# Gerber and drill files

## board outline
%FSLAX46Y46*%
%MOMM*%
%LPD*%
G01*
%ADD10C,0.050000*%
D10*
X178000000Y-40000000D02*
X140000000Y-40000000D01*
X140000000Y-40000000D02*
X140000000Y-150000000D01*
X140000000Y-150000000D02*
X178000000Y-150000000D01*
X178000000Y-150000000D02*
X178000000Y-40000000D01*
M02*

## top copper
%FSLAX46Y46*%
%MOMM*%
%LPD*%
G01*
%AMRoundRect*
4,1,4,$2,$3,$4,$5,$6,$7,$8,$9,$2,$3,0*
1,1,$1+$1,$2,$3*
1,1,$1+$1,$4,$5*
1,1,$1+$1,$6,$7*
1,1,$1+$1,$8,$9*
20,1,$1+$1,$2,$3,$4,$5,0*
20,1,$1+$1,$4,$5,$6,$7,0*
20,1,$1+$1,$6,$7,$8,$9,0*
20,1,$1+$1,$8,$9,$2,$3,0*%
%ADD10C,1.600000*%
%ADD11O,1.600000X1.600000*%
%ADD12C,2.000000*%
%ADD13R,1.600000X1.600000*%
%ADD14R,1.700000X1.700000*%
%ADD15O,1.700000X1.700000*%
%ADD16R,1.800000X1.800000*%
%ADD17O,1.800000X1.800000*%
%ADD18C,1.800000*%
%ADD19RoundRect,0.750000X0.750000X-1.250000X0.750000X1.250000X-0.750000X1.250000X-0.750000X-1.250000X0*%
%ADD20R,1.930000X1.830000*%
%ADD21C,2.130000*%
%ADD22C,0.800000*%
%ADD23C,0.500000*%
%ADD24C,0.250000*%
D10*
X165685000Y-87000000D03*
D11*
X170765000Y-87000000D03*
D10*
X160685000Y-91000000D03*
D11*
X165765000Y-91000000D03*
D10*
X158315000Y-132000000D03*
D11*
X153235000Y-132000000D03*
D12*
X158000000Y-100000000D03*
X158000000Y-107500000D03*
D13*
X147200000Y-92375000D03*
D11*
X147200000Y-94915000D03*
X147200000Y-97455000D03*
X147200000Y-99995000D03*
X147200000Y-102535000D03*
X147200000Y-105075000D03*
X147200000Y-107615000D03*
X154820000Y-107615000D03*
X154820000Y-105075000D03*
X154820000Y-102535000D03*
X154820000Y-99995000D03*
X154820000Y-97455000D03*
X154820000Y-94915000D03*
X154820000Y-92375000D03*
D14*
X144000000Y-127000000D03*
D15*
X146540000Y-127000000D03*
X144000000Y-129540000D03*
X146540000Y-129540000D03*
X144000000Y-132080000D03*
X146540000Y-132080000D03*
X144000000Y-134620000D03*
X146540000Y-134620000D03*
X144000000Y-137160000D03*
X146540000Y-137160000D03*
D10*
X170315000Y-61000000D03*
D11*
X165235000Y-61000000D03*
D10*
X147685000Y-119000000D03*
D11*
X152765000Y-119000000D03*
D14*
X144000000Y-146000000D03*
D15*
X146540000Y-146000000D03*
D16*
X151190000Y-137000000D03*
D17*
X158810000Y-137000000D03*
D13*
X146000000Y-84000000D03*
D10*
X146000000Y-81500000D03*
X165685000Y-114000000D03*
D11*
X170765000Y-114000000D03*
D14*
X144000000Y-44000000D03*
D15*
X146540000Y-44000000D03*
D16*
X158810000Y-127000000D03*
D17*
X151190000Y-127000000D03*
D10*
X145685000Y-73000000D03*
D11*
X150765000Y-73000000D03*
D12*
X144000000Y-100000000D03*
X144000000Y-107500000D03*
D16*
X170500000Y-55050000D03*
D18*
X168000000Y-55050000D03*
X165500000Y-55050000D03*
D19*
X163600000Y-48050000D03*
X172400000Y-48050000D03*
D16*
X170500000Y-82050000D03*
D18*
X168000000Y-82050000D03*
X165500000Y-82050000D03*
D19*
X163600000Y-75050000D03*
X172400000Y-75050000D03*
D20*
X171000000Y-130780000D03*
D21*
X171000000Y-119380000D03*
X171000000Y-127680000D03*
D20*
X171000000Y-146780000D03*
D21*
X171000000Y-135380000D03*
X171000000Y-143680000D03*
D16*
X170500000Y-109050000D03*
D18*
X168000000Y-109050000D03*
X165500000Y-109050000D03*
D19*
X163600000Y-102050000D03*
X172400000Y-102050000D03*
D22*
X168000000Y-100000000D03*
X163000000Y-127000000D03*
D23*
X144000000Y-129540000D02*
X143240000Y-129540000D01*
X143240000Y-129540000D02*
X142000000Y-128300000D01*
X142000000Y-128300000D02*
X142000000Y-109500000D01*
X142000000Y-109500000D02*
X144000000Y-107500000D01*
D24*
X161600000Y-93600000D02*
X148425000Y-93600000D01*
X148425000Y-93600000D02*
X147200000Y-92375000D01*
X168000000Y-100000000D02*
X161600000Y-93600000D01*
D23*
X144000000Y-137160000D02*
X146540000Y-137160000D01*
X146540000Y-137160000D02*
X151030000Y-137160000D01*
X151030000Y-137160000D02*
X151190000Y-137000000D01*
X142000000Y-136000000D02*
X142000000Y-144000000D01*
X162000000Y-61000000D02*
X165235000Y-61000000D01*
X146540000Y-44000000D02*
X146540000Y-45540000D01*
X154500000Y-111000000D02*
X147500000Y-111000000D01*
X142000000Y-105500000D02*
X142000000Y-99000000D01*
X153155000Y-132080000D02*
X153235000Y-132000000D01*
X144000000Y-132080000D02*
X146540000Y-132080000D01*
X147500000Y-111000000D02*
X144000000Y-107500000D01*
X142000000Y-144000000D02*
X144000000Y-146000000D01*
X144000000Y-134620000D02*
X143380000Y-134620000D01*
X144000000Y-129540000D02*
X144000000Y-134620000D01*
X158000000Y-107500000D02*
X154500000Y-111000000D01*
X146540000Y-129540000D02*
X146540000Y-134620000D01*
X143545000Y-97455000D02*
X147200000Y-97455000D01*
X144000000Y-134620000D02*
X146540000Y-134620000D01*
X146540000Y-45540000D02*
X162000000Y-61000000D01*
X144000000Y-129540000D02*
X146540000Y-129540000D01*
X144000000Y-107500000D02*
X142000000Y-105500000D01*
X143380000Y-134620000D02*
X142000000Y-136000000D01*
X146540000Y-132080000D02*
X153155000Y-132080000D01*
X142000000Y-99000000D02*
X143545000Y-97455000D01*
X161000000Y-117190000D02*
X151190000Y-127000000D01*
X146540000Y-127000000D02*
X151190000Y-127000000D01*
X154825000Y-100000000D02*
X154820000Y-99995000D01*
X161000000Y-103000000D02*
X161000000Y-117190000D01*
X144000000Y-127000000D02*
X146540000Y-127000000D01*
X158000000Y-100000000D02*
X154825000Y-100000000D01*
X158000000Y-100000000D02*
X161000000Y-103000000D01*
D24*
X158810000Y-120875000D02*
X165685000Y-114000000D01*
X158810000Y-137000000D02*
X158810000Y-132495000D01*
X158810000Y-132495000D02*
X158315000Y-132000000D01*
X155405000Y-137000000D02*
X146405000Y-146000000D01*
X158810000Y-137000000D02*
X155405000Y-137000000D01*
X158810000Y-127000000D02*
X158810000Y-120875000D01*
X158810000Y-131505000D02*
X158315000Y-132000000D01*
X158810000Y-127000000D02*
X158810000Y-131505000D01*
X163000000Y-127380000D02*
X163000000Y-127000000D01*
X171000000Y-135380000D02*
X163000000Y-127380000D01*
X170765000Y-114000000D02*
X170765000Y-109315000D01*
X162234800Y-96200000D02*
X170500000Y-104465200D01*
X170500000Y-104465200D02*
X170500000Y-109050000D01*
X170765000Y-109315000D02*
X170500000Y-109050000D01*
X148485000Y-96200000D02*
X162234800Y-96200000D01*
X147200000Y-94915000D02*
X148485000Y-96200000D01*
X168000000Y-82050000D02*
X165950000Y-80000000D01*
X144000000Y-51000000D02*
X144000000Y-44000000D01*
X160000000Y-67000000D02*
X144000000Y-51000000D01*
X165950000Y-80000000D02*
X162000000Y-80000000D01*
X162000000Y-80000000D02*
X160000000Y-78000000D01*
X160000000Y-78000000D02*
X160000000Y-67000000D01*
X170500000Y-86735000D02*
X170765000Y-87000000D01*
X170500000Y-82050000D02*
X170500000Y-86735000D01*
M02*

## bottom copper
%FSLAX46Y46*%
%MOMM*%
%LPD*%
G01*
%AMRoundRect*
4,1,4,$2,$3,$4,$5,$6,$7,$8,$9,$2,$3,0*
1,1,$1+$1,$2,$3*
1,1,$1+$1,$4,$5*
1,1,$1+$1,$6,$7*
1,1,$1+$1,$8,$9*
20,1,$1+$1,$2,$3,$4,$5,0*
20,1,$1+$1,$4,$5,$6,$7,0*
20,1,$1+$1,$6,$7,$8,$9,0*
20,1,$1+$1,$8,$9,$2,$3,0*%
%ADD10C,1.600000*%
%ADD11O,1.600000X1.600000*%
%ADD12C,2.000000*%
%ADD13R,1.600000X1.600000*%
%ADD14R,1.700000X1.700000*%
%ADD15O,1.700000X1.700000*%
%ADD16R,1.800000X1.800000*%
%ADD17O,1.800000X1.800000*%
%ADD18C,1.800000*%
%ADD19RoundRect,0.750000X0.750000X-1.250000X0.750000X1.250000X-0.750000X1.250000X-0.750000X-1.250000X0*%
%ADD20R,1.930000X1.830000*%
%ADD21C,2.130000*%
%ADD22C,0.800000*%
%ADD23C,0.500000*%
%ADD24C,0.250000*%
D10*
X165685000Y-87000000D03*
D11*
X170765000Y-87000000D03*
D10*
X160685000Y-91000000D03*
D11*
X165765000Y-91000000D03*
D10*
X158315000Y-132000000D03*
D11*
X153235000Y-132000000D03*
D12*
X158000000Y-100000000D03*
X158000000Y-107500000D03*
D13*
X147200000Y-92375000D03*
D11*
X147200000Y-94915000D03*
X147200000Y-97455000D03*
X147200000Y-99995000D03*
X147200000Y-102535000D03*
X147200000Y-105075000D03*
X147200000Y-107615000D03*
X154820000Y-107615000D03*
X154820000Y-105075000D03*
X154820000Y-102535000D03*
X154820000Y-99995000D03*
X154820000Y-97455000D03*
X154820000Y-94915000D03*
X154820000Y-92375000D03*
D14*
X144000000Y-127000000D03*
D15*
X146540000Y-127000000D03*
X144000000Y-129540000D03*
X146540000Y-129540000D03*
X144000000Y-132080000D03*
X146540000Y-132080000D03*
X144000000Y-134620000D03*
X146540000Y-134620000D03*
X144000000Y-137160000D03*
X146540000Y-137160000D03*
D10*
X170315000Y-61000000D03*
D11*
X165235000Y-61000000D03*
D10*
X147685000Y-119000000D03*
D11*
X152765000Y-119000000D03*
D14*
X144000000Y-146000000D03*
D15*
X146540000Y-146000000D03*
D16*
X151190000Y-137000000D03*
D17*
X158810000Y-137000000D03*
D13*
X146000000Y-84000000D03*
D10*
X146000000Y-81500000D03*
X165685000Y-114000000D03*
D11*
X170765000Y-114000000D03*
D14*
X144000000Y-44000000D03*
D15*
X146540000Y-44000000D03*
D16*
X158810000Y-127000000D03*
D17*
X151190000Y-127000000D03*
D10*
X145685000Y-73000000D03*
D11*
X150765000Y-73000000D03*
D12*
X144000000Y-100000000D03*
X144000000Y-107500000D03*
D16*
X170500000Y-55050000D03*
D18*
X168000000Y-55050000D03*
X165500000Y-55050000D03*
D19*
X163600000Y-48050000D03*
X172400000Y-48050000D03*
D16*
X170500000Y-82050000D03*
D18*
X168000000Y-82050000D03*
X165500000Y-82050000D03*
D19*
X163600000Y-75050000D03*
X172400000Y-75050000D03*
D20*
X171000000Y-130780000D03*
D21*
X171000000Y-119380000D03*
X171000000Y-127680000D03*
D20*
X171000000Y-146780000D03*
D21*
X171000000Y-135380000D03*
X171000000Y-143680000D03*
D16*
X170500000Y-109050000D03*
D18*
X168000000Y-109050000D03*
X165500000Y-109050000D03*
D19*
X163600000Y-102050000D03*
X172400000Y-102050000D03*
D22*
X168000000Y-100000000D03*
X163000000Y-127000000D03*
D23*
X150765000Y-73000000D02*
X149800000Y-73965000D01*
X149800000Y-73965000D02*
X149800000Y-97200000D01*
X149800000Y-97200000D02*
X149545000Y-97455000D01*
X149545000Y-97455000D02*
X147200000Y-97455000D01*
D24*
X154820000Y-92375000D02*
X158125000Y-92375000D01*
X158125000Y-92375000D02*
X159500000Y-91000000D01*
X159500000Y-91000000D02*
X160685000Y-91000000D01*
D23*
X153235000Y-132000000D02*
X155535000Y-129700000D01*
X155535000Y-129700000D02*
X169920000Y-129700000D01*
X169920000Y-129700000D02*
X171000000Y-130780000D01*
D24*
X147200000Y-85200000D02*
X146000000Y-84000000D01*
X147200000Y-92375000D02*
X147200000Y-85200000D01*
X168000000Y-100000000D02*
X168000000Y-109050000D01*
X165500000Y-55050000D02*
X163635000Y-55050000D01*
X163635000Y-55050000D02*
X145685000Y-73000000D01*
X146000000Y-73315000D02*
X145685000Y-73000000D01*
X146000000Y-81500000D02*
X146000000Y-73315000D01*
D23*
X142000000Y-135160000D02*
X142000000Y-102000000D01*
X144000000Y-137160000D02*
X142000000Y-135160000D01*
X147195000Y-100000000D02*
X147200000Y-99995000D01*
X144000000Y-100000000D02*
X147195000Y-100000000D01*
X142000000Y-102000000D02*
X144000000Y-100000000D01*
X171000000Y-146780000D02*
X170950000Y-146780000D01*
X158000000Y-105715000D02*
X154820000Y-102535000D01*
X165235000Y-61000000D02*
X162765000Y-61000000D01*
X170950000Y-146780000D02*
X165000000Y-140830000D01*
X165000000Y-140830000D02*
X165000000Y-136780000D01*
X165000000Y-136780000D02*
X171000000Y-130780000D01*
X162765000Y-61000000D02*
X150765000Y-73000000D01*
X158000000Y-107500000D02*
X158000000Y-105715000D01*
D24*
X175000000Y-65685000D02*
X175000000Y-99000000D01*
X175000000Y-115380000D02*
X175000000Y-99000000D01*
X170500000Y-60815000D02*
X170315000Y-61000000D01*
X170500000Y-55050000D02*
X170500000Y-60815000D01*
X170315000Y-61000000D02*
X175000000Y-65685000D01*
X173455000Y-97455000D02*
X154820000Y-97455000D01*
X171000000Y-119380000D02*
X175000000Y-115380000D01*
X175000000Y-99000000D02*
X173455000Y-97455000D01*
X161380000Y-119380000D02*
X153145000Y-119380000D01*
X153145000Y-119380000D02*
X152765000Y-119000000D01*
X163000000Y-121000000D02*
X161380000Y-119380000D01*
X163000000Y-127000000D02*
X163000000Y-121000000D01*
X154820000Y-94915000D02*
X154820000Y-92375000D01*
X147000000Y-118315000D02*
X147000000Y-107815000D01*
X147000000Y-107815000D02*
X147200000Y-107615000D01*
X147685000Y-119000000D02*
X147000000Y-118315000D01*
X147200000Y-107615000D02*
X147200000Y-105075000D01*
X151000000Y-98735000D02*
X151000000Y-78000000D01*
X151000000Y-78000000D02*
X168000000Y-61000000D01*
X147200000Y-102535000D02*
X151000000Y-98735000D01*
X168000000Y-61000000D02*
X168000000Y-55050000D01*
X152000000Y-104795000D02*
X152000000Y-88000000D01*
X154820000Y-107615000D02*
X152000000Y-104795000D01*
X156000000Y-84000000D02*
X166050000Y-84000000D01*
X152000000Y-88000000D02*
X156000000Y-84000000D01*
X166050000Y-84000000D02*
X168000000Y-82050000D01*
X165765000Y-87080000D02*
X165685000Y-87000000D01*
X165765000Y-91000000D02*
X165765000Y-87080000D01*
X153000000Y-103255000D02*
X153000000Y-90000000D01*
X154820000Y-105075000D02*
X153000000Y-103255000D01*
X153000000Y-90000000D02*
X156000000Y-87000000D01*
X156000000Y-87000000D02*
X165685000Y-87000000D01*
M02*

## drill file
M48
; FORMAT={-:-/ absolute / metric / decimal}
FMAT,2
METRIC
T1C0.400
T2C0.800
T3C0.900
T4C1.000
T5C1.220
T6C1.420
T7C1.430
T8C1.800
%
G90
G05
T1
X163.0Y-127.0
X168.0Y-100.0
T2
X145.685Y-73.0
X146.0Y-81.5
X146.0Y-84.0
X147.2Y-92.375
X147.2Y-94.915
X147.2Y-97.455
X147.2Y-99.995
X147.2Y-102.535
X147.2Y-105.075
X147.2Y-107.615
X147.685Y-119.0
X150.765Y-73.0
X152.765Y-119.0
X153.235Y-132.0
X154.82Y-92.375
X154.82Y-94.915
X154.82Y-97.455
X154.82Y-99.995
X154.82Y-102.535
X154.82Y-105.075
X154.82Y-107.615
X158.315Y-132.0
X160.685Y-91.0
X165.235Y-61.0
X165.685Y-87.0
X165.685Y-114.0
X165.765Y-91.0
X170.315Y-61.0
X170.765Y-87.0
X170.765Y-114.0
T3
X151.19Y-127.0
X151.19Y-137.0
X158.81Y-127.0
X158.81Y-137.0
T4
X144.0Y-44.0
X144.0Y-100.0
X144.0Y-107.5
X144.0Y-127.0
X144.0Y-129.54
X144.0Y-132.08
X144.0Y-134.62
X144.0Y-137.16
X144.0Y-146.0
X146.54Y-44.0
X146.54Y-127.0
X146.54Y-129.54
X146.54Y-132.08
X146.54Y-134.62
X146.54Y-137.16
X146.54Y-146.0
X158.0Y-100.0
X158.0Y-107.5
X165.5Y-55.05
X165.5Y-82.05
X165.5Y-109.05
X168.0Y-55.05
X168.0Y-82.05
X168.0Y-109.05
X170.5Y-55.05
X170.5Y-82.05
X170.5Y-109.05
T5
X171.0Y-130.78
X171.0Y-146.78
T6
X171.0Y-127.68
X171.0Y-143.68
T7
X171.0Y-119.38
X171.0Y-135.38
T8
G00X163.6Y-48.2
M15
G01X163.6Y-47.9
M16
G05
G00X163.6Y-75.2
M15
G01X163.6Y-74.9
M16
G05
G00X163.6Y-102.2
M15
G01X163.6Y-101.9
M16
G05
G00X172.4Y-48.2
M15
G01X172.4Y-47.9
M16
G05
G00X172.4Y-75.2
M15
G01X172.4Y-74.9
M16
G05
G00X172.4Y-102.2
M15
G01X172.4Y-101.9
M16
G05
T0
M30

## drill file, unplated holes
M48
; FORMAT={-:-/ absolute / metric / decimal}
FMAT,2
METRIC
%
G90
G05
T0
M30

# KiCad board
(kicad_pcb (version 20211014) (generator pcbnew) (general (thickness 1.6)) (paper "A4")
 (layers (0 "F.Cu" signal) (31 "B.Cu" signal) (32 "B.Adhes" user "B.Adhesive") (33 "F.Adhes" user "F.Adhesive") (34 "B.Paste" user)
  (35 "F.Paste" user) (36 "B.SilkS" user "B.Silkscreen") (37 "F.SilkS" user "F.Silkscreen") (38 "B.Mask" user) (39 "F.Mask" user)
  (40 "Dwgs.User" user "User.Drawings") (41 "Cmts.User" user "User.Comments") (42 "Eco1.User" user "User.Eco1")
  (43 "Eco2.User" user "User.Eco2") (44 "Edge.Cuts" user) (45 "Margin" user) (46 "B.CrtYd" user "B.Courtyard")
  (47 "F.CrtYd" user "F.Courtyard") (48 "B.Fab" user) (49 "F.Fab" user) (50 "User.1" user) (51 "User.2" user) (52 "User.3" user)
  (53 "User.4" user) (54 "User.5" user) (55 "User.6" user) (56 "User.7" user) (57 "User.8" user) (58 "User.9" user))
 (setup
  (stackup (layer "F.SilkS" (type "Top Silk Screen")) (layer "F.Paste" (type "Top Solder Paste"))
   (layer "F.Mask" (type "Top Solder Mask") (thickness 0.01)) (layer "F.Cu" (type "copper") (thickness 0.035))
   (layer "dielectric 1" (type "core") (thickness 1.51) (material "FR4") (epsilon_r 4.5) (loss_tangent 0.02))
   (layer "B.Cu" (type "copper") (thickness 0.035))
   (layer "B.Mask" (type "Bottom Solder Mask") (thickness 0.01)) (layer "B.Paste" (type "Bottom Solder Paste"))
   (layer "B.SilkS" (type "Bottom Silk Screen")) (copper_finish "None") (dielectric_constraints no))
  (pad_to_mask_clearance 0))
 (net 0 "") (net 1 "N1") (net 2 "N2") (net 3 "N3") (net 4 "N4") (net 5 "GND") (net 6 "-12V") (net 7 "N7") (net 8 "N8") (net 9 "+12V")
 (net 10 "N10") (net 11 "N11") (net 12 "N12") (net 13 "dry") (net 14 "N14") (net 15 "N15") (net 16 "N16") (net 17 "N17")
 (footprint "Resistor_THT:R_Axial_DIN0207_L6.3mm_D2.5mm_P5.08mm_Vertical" (layer "F.Cu") (at 165.685 87)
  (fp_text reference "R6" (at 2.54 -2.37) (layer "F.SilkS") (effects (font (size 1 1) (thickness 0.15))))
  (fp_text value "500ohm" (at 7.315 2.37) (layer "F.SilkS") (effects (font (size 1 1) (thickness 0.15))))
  (pad "1" thru_hole circle (at 0 0) (size 1.6 1.6) (drill 0.8) (layers *.Cu *.Mask) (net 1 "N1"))
  (pad "2" thru_hole oval (at 5.08 0) (size 1.6 1.6) (drill 0.8) (layers *.Cu *.Mask) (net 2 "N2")))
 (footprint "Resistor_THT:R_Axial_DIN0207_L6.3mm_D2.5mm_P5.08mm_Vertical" (layer "F.Cu") (at 160.685 91)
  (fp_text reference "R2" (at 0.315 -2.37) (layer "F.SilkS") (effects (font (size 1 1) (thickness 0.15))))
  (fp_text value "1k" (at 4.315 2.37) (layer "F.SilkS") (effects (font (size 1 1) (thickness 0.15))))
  (pad "1" thru_hole circle (at 0 0) (size 1.6 1.6) (drill 0.8) (layers *.Cu *.Mask) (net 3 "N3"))
  (pad "2" thru_hole oval (at 5.08 0) (size 1.6 1.6) (drill 0.8) (layers *.Cu *.Mask) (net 1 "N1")))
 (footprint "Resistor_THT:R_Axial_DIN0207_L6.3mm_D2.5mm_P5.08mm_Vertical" (layer "F.Cu") (at 158.315 132 180)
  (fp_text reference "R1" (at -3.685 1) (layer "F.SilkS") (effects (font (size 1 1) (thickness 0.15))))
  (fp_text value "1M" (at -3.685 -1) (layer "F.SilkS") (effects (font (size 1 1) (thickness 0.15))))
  (pad "1" thru_hole circle (at 0 0 180) (size 1.6 1.6) (drill 0.8) (layers *.Cu *.Mask) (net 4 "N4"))
  (pad "2" thru_hole oval (at 5.08 0 180) (size 1.6 1.6) (drill 0.8) (layers *.Cu *.Mask) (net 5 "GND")))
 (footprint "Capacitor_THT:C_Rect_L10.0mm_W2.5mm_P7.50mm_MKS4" (layer "F.Cu") (at 158 100 -90)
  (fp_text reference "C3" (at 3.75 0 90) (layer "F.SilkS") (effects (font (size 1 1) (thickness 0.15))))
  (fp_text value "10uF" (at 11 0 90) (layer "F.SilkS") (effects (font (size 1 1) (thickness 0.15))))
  (pad "1" thru_hole circle (at 0 0 270) (size 2 2) (drill 1) (layers *.Cu *.Mask) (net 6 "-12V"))
  (pad "2" thru_hole circle (at 7.5 0 270) (size 2 2) (drill 1) (layers *.Cu *.Mask) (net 5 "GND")))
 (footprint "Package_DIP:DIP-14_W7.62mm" (layer "F.Cu") (at 147.2 92.375)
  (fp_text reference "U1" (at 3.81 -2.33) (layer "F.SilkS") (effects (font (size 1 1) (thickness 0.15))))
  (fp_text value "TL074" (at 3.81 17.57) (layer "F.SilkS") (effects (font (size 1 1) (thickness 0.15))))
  (pad "1" thru_hole rect (at 0 0) (size 1.6 1.6) (drill 0.8) (layers *.Cu *.Mask) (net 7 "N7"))
  (pad "2" thru_hole oval (at 0 2.54) (size 1.6 1.6) (drill 0.8) (layers *.Cu *.Mask) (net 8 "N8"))
  (pad "3" thru_hole oval (at 0 5.08) (size 1.6 1.6) (drill 0.8) (layers *.Cu *.Mask) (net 5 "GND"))
  (pad "4" thru_hole oval (at 0 7.62) (size 1.6 1.6) (drill 0.8) (layers *.Cu *.Mask) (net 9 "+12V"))
  (pad "5" thru_hole oval (at 0 10.16) (size 1.6 1.6) (drill 0.8) (layers *.Cu *.Mask) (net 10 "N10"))
  (pad "6" thru_hole oval (at 0 12.7) (size 1.6 1.6) (drill 0.8) (layers *.Cu *.Mask) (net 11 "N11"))
  (pad "7" thru_hole oval (at 0 15.24) (size 1.6 1.6) (drill 0.8) (layers *.Cu *.Mask) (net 11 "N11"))
  (pad "8" thru_hole oval (at 7.62 15.24) (size 1.6 1.6) (drill 0.8) (layers *.Cu *.Mask) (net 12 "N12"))
  (pad "9" thru_hole oval (at 7.62 12.7) (size 1.6 1.6) (drill 0.8) (layers *.Cu *.Mask) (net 1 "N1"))
  (pad "10" thru_hole oval (at 7.62 10.16) (size 1.6 1.6) (drill 0.8) (layers *.Cu *.Mask) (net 5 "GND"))
  (pad "11" thru_hole oval (at 7.62 7.62) (size 1.6 1.6) (drill 0.8) (layers *.Cu *.Mask) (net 6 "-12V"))
  (pad "12" thru_hole oval (at 7.62 5.08) (size 1.6 1.6) (drill 0.8) (layers *.Cu *.Mask) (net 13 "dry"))
  (pad "13" thru_hole oval (at 7.62 2.54) (size 1.6 1.6) (drill 0.8) (layers *.Cu *.Mask) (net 3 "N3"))
  (pad "14" thru_hole oval (at 7.62 0) (size 1.6 1.6) (drill 0.8) (layers *.Cu *.Mask) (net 3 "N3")))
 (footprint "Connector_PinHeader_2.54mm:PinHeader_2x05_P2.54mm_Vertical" (layer "F.Cu") (at 144 127)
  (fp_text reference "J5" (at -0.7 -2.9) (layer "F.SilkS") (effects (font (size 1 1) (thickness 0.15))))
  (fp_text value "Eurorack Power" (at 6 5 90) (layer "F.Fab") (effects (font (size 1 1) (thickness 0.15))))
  (pad "1" thru_hole rect (at 0 0) (size 1.7 1.7) (drill 1) (layers *.Cu *.Mask) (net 6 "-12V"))
  (pad "2" thru_hole oval (at 2.54 0) (size 1.7 1.7) (drill 1) (layers *.Cu *.Mask) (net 6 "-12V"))
  (pad "3" thru_hole oval (at 0 2.54) (size 1.7 1.7) (drill 1) (layers *.Cu *.Mask) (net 5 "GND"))
  (pad "4" thru_hole oval (at 2.54 2.54) (size 1.7 1.7) (drill 1) (layers *.Cu *.Mask) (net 5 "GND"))
  (pad "5" thru_hole oval (at 0 5.08) (size 1.7 1.7) (drill 1) (layers *.Cu *.Mask) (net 5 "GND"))
  (pad "6" thru_hole oval (at 2.54 5.08) (size 1.7 1.7) (drill 1) (layers *.Cu *.Mask) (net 5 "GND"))
  (pad "7" thru_hole oval (at 0 7.62) (size 1.7 1.7) (drill 1) (layers *.Cu *.Mask) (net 5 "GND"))
  (pad "8" thru_hole oval (at 2.54 7.62) (size 1.7 1.7) (drill 1) (layers *.Cu *.Mask) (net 5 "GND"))
  (pad "9" thru_hole oval (at 0 10.16) (size 1.7 1.7) (drill 1) (layers *.Cu *.Mask) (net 9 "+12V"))
  (pad "10" thru_hole oval (at 2.54 10.16) (size 1.7 1.7) (drill 1) (layers *.Cu *.Mask) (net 9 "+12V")))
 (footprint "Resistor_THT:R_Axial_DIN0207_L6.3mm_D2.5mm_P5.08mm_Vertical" (layer "F.Cu") (at 170.315 61 180)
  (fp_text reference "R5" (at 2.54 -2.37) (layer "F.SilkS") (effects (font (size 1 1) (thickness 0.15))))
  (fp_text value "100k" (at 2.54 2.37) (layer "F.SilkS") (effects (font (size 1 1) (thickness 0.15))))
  (pad "1" thru_hole circle (at 0 0 180) (size 1.6 1.6) (drill 0.8) (layers *.Cu *.Mask) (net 13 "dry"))
  (pad "2" thru_hole oval (at 5.08 0 180) (size 1.6 1.6) (drill 0.8) (layers *.Cu *.Mask) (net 5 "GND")))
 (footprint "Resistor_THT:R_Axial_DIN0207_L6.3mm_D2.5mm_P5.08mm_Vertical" (layer "F.Cu") (at 147.685 119)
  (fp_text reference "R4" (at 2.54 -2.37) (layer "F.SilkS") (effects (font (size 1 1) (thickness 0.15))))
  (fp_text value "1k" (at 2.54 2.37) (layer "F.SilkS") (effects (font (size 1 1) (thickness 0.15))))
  (pad "1" thru_hole circle (at 0 0) (size 1.6 1.6) (drill 0.8) (layers *.Cu *.Mask) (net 11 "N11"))
  (pad "2" thru_hole oval (at 5.08 0) (size 1.6 1.6) (drill 0.8) (layers *.Cu *.Mask) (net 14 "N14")))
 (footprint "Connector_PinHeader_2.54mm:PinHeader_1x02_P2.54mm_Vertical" (layer "F.Cu") (at 144 146 90)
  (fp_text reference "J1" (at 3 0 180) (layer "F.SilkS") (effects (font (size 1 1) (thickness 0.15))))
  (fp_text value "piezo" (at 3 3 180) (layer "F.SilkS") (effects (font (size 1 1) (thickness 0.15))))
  (pad "1" thru_hole rect (at 0 0 90) (size 1.7 1.7) (drill 1) (layers *.Cu *.Mask) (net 5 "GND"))
  (pad "2" thru_hole oval (at 0 2.54 90) (size 1.7 1.7) (drill 1) (layers *.Cu *.Mask) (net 4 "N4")))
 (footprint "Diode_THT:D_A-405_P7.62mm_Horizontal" (layer "F.Cu") (at 151.19 137)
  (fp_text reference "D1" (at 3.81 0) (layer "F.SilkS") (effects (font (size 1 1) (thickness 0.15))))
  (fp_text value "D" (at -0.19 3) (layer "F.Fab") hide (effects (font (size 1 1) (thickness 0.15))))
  (pad "1" thru_hole rect (at 0 0) (size 1.8 1.8) (drill 0.9) (layers *.Cu *.Mask) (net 9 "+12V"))
  (pad "2" thru_hole oval (at 7.62 0) (size 1.8 1.8) (drill 0.9) (layers *.Cu *.Mask) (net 4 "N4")))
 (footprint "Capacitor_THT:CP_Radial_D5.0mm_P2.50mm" (layer "F.Cu") (at 146 84 90)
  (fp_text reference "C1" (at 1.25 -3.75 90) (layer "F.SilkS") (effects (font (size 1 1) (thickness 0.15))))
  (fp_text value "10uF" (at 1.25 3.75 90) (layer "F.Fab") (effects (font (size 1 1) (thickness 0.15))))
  (pad "1" thru_hole rect (at 0 0 90) (size 1.6 1.6) (drill 0.8) (layers *.Cu *.Mask) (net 7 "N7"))
  (pad "2" thru_hole circle (at 2.5 0 90) (size 1.6 1.6) (drill 0.8) (layers *.Cu *.Mask) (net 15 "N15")))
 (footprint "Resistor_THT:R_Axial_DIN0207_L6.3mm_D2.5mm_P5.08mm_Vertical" (layer "F.Cu") (at 165.685 114)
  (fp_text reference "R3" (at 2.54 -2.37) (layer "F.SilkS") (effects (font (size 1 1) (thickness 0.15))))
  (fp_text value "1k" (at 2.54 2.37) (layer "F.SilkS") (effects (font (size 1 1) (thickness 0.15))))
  (pad "1" thru_hole circle (at 0 0) (size 1.6 1.6) (drill 0.8) (layers *.Cu *.Mask) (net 4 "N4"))
  (pad "2" thru_hole oval (at 5.08 0) (size 1.6 1.6) (drill 0.8) (layers *.Cu *.Mask) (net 8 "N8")))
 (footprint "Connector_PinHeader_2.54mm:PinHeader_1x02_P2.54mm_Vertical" (layer "F.Cu") (at 144 44 90)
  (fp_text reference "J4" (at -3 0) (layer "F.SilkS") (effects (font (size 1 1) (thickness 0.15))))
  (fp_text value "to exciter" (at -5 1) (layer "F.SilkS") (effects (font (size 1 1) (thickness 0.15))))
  (pad "1" thru_hole rect (at 0 0 90) (size 1.7 1.7) (drill 1) (layers *.Cu *.Mask) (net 12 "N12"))
  (pad "2" thru_hole oval (at 0 2.54 90) (size 1.7 1.7) (drill 1) (layers *.Cu *.Mask) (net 5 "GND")))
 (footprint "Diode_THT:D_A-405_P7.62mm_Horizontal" (layer "F.Cu") (at 158.81 127 180)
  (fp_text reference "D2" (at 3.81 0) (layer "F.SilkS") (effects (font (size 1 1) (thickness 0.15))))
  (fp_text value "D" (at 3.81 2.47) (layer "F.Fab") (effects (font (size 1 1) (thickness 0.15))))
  (pad "1" thru_hole rect (at 0 0 180) (size 1.8 1.8) (drill 0.9) (layers *.Cu *.Mask) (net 4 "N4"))
  (pad "2" thru_hole oval (at 7.62 0 180) (size 1.8 1.8) (drill 0.9) (layers *.Cu *.Mask) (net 6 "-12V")))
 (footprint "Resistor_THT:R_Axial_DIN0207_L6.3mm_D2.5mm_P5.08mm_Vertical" (layer "F.Cu") (at 145.685 73)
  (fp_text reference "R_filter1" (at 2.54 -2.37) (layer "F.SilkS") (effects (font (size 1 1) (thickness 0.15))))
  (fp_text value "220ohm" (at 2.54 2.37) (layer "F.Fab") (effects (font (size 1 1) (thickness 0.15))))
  (pad "1" thru_hole circle (at 0 0) (size 1.6 1.6) (drill 0.8) (layers *.Cu *.Mask) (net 15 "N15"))
  (pad "2" thru_hole oval (at 5.08 0) (size 1.6 1.6) (drill 0.8) (layers *.Cu *.Mask) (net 5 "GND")))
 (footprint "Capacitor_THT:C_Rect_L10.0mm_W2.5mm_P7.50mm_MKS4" (layer "F.Cu") (at 144 100 -90)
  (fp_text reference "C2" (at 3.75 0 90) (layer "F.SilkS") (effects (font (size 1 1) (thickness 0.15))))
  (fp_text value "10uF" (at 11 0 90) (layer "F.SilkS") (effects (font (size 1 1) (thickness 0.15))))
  (pad "1" thru_hole circle (at 0 0 270) (size 2 2) (drill 1) (layers *.Cu *.Mask) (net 9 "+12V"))
  (pad "2" thru_hole circle (at 7.5 0 270) (size 2 2) (drill 1) (layers *.Cu *.Mask) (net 5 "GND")))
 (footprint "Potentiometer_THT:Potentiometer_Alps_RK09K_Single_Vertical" (layer "B.Cu") (at 170.5 55.05 90)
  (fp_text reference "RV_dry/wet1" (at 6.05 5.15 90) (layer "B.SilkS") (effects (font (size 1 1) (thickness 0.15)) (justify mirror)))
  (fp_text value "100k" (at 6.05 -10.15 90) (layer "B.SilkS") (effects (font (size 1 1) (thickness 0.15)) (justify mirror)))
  (pad "1" thru_hole rect (at 0 0 90) (size 1.8 1.8) (drill 1) (layers *.Cu *.Mask) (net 13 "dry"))
  (pad "2" thru_hole circle (at 0 -2.5 90) (size 1.8 1.8) (drill 1) (layers *.Cu *.Mask) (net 10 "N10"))
  (pad "3" thru_hole circle (at 0 -5 90) (size 1.8 1.8) (drill 1) (layers *.Cu *.Mask) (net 15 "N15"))
  (pad "MP" thru_hole roundrect (at 7 -6.9 90) (size 4 3) (drill oval 2.1 1.8) (layers *.Cu *.Mask) (roundrect_rratio 0.25))
  (pad "MP" thru_hole roundrect (at 7 1.9 90) (size 4 3) (drill oval 2.1 1.8) (layers *.Cu *.Mask) (roundrect_rratio 0.25)))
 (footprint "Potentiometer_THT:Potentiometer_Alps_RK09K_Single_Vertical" (layer "B.Cu") (at 170.5 82.05 90)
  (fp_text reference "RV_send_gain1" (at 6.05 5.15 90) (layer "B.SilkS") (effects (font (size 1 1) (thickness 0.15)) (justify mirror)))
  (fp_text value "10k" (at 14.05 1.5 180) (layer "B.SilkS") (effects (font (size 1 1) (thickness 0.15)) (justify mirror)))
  (pad "1" thru_hole rect (at 0 0 90) (size 1.8 1.8) (drill 1) (layers *.Cu *.Mask) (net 2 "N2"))
  (pad "2" thru_hole circle (at 0 -2.5 90) (size 1.8 1.8) (drill 1) (layers *.Cu *.Mask) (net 12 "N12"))
  (pad "3" thru_hole circle (at 0 -5 90) (size 1.8 1.8) (drill 1) (layers *.Cu *.Mask))
  (pad "MP" thru_hole roundrect (at 7 -6.9 90) (size 4 3) (drill oval 2.1 1.8) (layers *.Cu *.Mask) (roundrect_rratio 0.25))
  (pad "MP" thru_hole roundrect (at 7 1.9 90) (size 4 3) (drill oval 2.1 1.8) (layers *.Cu *.Mask) (roundrect_rratio 0.25)))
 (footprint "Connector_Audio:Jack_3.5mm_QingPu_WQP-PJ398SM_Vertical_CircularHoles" (layer "B.Cu") (at 171 130.78)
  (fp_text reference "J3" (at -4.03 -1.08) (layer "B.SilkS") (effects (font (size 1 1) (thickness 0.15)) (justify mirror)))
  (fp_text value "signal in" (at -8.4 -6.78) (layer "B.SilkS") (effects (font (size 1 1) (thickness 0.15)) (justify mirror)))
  (pad "S" thru_hole rect (at 0 0 180) (size 1.93 1.83) (drill 1.22) (layers *.Cu *.Mask) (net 5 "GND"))
  (pad "T" thru_hole circle (at 0 -11.4 180) (size 2.13 2.13) (drill 1.43) (layers *.Cu *.Mask) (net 13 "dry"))
  (pad "TN" thru_hole circle (at 0 -3.1 180) (size 2.13 2.13) (drill 1.42) (layers *.Cu *.Mask) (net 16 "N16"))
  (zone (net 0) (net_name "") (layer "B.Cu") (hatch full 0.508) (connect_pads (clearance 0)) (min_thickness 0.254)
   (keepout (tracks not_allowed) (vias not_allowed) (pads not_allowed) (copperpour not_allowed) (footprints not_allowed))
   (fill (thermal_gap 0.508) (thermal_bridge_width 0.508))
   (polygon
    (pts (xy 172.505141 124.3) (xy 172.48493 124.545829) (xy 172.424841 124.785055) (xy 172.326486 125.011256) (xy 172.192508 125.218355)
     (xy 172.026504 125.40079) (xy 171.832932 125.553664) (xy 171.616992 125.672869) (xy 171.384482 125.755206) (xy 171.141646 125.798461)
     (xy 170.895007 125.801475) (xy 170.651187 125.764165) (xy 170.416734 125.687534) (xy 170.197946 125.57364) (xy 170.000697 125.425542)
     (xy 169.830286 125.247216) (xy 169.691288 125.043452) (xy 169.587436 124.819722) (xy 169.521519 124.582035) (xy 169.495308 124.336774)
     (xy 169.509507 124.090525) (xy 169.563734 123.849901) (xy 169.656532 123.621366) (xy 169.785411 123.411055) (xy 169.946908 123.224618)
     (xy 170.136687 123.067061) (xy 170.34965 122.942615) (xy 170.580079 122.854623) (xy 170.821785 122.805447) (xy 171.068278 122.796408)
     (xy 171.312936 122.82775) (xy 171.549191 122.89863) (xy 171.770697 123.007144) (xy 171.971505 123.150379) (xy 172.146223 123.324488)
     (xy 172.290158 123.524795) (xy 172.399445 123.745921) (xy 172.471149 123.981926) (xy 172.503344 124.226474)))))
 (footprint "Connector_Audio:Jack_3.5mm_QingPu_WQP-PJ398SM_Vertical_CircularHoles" (layer "B.Cu") (at 171 146.78)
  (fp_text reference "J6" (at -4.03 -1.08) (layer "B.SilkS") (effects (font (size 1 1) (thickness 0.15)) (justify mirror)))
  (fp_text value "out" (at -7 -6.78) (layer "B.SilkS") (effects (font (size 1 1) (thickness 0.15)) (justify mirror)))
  (pad "S" thru_hole rect (at 0 0 180) (size 1.93 1.83) (drill 1.22) (layers *.Cu *.Mask) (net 5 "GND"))
  (pad "T" thru_hole circle (at 0 -11.4 180) (size 2.13 2.13) (drill 1.43) (layers *.Cu *.Mask) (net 14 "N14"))
  (pad "TN" thru_hole circle (at 0 -3.1 180) (size 2.13 2.13) (drill 1.42) (layers *.Cu *.Mask) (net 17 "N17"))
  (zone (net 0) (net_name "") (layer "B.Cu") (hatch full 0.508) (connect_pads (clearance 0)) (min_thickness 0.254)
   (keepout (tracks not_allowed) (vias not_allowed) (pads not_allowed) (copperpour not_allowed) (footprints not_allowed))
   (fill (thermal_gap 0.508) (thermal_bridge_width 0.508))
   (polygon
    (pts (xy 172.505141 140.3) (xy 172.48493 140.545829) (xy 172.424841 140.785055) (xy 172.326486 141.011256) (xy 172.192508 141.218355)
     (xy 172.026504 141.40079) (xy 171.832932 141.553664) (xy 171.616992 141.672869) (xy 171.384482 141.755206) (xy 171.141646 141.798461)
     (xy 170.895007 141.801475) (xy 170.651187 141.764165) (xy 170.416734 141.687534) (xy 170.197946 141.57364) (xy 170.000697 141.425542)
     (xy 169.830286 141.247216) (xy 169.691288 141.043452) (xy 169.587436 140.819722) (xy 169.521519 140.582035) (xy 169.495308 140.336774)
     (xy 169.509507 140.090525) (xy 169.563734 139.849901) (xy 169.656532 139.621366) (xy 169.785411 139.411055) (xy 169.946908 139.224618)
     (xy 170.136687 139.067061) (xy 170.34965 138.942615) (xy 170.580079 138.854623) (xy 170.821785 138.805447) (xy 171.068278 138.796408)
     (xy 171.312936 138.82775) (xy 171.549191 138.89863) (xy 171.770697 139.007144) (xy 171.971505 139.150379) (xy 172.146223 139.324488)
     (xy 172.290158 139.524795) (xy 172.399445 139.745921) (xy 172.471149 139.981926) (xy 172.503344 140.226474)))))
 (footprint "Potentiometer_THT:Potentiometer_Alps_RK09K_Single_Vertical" (layer "B.Cu") (at 170.5 109.05 90)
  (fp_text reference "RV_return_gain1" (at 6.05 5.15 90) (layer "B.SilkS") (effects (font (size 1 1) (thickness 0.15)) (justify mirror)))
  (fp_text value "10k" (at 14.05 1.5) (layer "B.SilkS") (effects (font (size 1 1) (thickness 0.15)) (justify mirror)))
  (pad "1" thru_hole rect (at 0 0 90) (size 1.8 1.8) (drill 1) (layers *.Cu *.Mask) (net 8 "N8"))
  (pad "2" thru_hole circle (at 0 -2.5 90) (size 1.8 1.8) (drill 1) (layers *.Cu *.Mask) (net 7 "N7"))
  (pad "3" thru_hole circle (at 0 -5 90) (size 1.8 1.8) (drill 1) (layers *.Cu *.Mask))
  (pad "MP" thru_hole roundrect (at 7 -6.9 90) (size 4 3) (drill oval 2.1 1.8) (layers *.Cu *.Mask) (roundrect_rratio 0.25))
  (pad "MP" thru_hole roundrect (at 7 1.9 90) (size 4 3) (drill oval 2.1 1.8) (layers *.Cu *.Mask) (roundrect_rratio 0.25)))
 (gr_rect (start 178 40) (end 140 150) (layer "Edge.Cuts") (width 0.05) (fill none))
 (segment (start 161.6 93.6) (end 148.425 93.6) (width 0.25) (layer "F.Cu") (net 7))
 (segment (start 148.425 93.6) (end 147.2 92.375) (width 0.25) (layer "F.Cu") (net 7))
 (segment (start 168 100) (end 161.6 93.6) (width 0.25) (layer "F.Cu") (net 7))
 (via (at 168 100) (size 0.8) (drill 0.4) (layers "F.Cu" "B.Cu") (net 7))
 (segment (start 147.2 85.2) (end 146 84) (width 0.25) (layer "B.Cu") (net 7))
 (segment (start 147.2 92.375) (end 147.2 85.2) (width 0.25) (layer "B.Cu") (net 7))
 (segment (start 168 100) (end 168 109.05) (width 0.25) (layer "B.Cu") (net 7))
 (segment (start 165.5 55.05) (end 163.635 55.05) (width 0.25) (layer "B.Cu") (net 15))
 (segment (start 163.635 55.05) (end 145.685 73) (width 0.25) (layer "B.Cu") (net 15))
 (segment (start 146 73.315) (end 145.685 73) (width 0.25) (layer "B.Cu") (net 15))
 (segment (start 146 81.5) (end 146 73.315) (width 0.25) (layer "B.Cu") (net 15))
 (segment (start 144 137.16) (end 146.54 137.16) (width 0.5) (layer "F.Cu") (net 9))
 (segment (start 146.54 137.16) (end 151.03 137.16) (width 0.5) (layer "F.Cu") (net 9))
 (segment (start 151.03 137.16) (end 151.19 137) (width 0.5) (layer "F.Cu") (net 9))
 (segment (start 142 135.16) (end 142 102) (width 0.5) (layer "B.Cu") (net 9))
 (segment (start 144 137.16) (end 142 135.16) (width 0.5) (layer "B.Cu") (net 9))
 (segment (start 147.195 100) (end 147.2 99.995) (width 0.5) (layer "B.Cu") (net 9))
 (segment (start 144 100) (end 147.195 100) (width 0.5) (layer "B.Cu") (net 9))
 (segment (start 142 102) (end 144 100) (width 0.5) (layer "B.Cu") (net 9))
 (segment (start 142 109.5) (end 144 107.5) (width 0.5) (layer "F.Cu") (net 5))
 (segment (start 142 136) (end 142 144) (width 0.5) (layer "F.Cu") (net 5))
 (segment (start 162 61) (end 165.235 61) (width 0.5) (layer "F.Cu") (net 5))
 (segment (start 146.54 44) (end 146.54 45.54) (width 0.5) (layer "F.Cu") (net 5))
 (segment (start 154.5 111) (end 147.5 111) (width 0.5) (layer "F.Cu") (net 5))
 (segment (start 142 105.5) (end 142 99) (width 0.5) (layer "F.Cu") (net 5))
 (segment (start 153.155 132.08) (end 153.235 132) (width 0.5) (layer "F.Cu") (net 5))
 (segment (start 144 132.08) (end 146.54 132.08) (width 0.5) (layer "F.Cu") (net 5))
 (segment (start 147.5 111) (end 144 107.5) (width 0.5) (layer "F.Cu") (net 5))
 (segment (start 142 144) (end 144 146) (width 0.5) (layer "F.Cu") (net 5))
 (segment (start 144 134.62) (end 143.38 134.62) (width 0.5) (layer "F.Cu") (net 5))
 (segment (start 144 129.54) (end 144 134.62) (width 0.5) (layer "F.Cu") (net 5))
 (segment (start 158 107.5) (end 154.5 111) (width 0.5) (layer "F.Cu") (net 5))
 (segment (start 146.54 129.54) (end 146.54 134.62) (width 0.5) (layer "F.Cu") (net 5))
 (segment (start 143.545 97.455) (end 147.2 97.455) (width 0.5) (layer "F.Cu") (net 5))
 (segment (start 144 134.62) (end 146.54 134.62) (width 0.5) (layer "F.Cu") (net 5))
 (segment (start 146.54 45.54) (end 162 61) (width 0.5) (layer "F.Cu") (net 5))
 (segment (start 144 129.54) (end 146.54 129.54) (width 0.5) (layer "F.Cu") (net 5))
 (segment (start 144 129.54) (end 143.24 129.54) (width 0.5) (layer "F.Cu") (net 5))
 (segment (start 144 107.5) (end 142 105.5) (width 0.5) (layer "F.Cu") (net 5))
 (segment (start 142 128.3) (end 142 109.5) (width 0.5) (layer "F.Cu") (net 5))
 (segment (start 143.38 134.62) (end 142 136) (width 0.5) (layer "F.Cu") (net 5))
 (segment (start 146.54 132.08) (end 153.155 132.08) (width 0.5) (layer "F.Cu") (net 5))
 (segment (start 142 99) (end 143.545 97.455) (width 0.5) (layer "F.Cu") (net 5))
 (segment (start 143.24 129.54) (end 142 128.3) (width 0.5) (layer "F.Cu") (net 5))
 (segment (start 171 146.78) (end 170.95 146.78) (width 0.5) (layer "B.Cu") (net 5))
 (segment (start 158 105.715) (end 154.82 102.535) (width 0.5) (layer "B.Cu") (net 5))
 (segment (start 165.235 61) (end 162.765 61) (width 0.5) (layer "B.Cu") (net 5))
 (segment (start 149.545 97.455) (end 147.2 97.455) (width 0.5) (layer "B.Cu") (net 5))
 (segment (start 149.8 97.2) (end 149.545 97.455) (width 0.5) (layer "B.Cu") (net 5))
 (segment (start 170.95 146.78) (end 165 140.83) (width 0.5) (layer "B.Cu") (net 5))
 (segment (start 165 140.83) (end 165 136.78) (width 0.5) (layer "B.Cu") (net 5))
 (segment (start 165 136.78) (end 171 130.78) (width 0.5) (layer "B.Cu") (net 5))
 (segment (start 155.535 129.7) (end 169.92 129.7) (width 0.5) (layer "B.Cu") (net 5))
 (segment (start 153.235 132) (end 155.535 129.7) (width 0.5) (layer "B.Cu") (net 5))
 (segment (start 150.765 73) (end 149.8 73.965) (width 0.5) (layer "B.Cu") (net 5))
 (segment (start 169.92 129.7) (end 171 130.78) (width 0.5) (layer "B.Cu") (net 5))
 (segment (start 149.8 73.965) (end 149.8 97.2) (width 0.5) (layer "B.Cu") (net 5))
 (segment (start 162.765 61) (end 150.765 73) (width 0.5) (layer "B.Cu") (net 5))
 (segment (start 158 107.5) (end 158 105.715) (width 0.5) (layer "B.Cu") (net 5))
 (segment (start 161 117.19) (end 151.19 127) (width 0.5) (layer "F.Cu") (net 6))
 (segment (start 146.54 127) (end 151.19 127) (width 0.5) (layer "F.Cu") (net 6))
 (segment (start 154.825 100) (end 154.82 99.995) (width 0.5) (layer "F.Cu") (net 6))
 (segment (start 161 103) (end 161 117.19) (width 0.5) (layer "F.Cu") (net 6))
 (segment (start 144 127) (end 146.54 127) (width 0.5) (layer "F.Cu") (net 6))
 (segment (start 158 100) (end 154.825 100) (width 0.5) (layer "F.Cu") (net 6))
 (segment (start 158 100) (end 161 103) (width 0.5) (layer "F.Cu") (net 6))
 (segment (start 158.81 120.875) (end 165.685 114) (width 0.25) (layer "F.Cu") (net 4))
 (segment (start 158.81 137) (end 158.81 132.495) (width 0.25) (layer "F.Cu") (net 4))
 (segment (start 158.81 132.495) (end 158.315 132) (width 0.25) (layer "F.Cu") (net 4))
 (segment (start 155.405 137) (end 146.405 146) (width 0.25) (layer "F.Cu") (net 4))
 (segment (start 158.81 137) (end 155.405 137) (width 0.25) (layer "F.Cu") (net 4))
 (segment (start 158.81 127) (end 158.81 120.875) (width 0.25) (layer "F.Cu") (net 4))
 (segment (start 158.81 131.505) (end 158.315 132) (width 0.25) (layer "F.Cu") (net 4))
 (segment (start 158.81 127) (end 158.81 131.505) (width 0.25) (layer "F.Cu") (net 4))
 (segment (start 175 65.685) (end 175 99) (width 0.25) (layer "B.Cu") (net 13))
 (segment (start 175 115.38) (end 175 99) (width 0.25) (layer "B.Cu") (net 13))
 (segment (start 170.5 60.815) (end 170.315 61) (width 0.25) (layer "B.Cu") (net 13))
 (segment (start 170.5 55.05) (end 170.5 60.815) (width 0.25) (layer "B.Cu") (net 13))
 (segment (start 170.315 61) (end 175 65.685) (width 0.25) (layer "B.Cu") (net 13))
 (segment (start 173.455 97.455) (end 154.82 97.455) (width 0.25) (layer "B.Cu") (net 13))
 (segment (start 171 119.38) (end 175 115.38) (width 0.25) (layer "B.Cu") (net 13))
 (segment (start 175 99) (end 173.455 97.455) (width 0.25) (layer "B.Cu") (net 13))
 (segment (start 163 127.38) (end 163 127) (width 0.25) (layer "F.Cu") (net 14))
 (segment (start 171 135.38) (end 163 127.38) (width 0.25) (layer "F.Cu") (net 14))
 (via (at 163 127) (size 0.8) (drill 0.4) (layers "F.Cu" "B.Cu") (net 14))
 (segment (start 161.38 119.38) (end 153.145 119.38) (width 0.25) (layer "B.Cu") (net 14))
 (segment (start 153.145 119.38) (end 152.765 119) (width 0.25) (layer "B.Cu") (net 14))
 (segment (start 163 121) (end 161.38 119.38) (width 0.25) (layer "B.Cu") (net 14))
 (segment (start 163 127) (end 163 121) (width 0.25) (layer "B.Cu") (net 14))
 (segment (start 154.82 94.915) (end 154.82 92.375) (width 0.25) (layer "B.Cu") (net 3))
 (segment (start 159.5 91) (end 160.685 91) (width 0.25) (layer "B.Cu") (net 3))
 (segment (start 154.82 92.375) (end 158.125 92.375) (width 0.25) (layer "B.Cu") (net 3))
 (segment (start 158.125 92.375) (end 159.5 91) (width 0.25) (layer "B.Cu") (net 3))
 (segment (start 170.765 114) (end 170.765 109.315) (width 0.25) (layer "F.Cu") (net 8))
 (segment (start 162.2348 96.2) (end 170.5 104.4652) (width 0.25) (layer "F.Cu") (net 8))
 (segment (start 170.5 104.4652) (end 170.5 109.05) (width 0.25) (layer "F.Cu") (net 8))
 (segment (start 170.765 109.315) (end 170.5 109.05) (width 0.25) (layer "F.Cu") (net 8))
 (segment (start 148.485 96.2) (end 162.2348 96.2) (width 0.25) (layer "F.Cu") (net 8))
 (segment (start 147.2 94.915) (end 148.485 96.2) (width 0.25) (layer "F.Cu") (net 8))
 (segment (start 147 118.315) (end 147 107.815) (width 0.25) (layer "B.Cu") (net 11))
 (segment (start 147 107.815) (end 147.2 107.615) (width 0.25) (layer "B.Cu") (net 11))
 (segment (start 147.685 119) (end 147 118.315) (width 0.25) (layer "B.Cu") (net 11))
 (segment (start 147.2 107.615) (end 147.2 105.075) (width 0.25) (layer "B.Cu") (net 11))
 (segment (start 151 98.735) (end 151 78) (width 0.25) (layer "B.Cu") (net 10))
 (segment (start 151 78) (end 168 61) (width 0.25) (layer "B.Cu") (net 10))
 (segment (start 147.2 102.535) (end 151 98.735) (width 0.25) (layer "B.Cu") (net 10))
 (segment (start 168 61) (end 168 55.05) (width 0.25) (layer "B.Cu") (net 10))
 (segment (start 168 82.05) (end 165.95 80) (width 0.25) (layer "F.Cu") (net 12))
 (segment (start 144 51) (end 144 44) (width 0.25) (layer "F.Cu") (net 12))
 (segment (start 160 67) (end 144 51) (width 0.25) (layer "F.Cu") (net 12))
 (segment (start 165.95 80) (end 162 80) (width 0.25) (layer "F.Cu") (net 12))
 (segment (start 162 80) (end 160 78) (width 0.25) (layer "F.Cu") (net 12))
 (segment (start 160 78) (end 160 67) (width 0.25) (layer "F.Cu") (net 12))
 (segment (start 152 104.795) (end 152 88) (width 0.25) (layer "B.Cu") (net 12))
 (segment (start 154.82 107.615) (end 152 104.795) (width 0.25) (layer "B.Cu") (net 12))
 (segment (start 156 84) (end 166.05 84) (width 0.25) (layer "B.Cu") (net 12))
 (segment (start 152 88) (end 156 84) (width 0.25) (layer "B.Cu") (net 12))
 (segment (start 166.05 84) (end 168 82.05) (width 0.25) (layer "B.Cu") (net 12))
 (segment (start 165.765 87.08) (end 165.685 87) (width 0.25) (layer "B.Cu") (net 1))
 (segment (start 165.765 91) (end 165.765 87.08) (width 0.25) (layer "B.Cu") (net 1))
 (segment (start 153 103.255) (end 153 90) (width 0.25) (layer "B.Cu") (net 1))
 (segment (start 154.82 105.075) (end 153 103.255) (width 0.25) (layer "B.Cu") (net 1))
 (segment (start 153 90) (end 156 87) (width 0.25) (layer "B.Cu") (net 1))
 (segment (start 156 87) (end 165.685 87) (width 0.25) (layer "B.Cu") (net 1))
 (segment (start 170.5 86.735) (end 170.765 87) (width 0.25) (layer "F.Cu") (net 2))
 (segment (start 170.5 82.05) (end 170.5 86.735) (width 0.25) (layer "F.Cu") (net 2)))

